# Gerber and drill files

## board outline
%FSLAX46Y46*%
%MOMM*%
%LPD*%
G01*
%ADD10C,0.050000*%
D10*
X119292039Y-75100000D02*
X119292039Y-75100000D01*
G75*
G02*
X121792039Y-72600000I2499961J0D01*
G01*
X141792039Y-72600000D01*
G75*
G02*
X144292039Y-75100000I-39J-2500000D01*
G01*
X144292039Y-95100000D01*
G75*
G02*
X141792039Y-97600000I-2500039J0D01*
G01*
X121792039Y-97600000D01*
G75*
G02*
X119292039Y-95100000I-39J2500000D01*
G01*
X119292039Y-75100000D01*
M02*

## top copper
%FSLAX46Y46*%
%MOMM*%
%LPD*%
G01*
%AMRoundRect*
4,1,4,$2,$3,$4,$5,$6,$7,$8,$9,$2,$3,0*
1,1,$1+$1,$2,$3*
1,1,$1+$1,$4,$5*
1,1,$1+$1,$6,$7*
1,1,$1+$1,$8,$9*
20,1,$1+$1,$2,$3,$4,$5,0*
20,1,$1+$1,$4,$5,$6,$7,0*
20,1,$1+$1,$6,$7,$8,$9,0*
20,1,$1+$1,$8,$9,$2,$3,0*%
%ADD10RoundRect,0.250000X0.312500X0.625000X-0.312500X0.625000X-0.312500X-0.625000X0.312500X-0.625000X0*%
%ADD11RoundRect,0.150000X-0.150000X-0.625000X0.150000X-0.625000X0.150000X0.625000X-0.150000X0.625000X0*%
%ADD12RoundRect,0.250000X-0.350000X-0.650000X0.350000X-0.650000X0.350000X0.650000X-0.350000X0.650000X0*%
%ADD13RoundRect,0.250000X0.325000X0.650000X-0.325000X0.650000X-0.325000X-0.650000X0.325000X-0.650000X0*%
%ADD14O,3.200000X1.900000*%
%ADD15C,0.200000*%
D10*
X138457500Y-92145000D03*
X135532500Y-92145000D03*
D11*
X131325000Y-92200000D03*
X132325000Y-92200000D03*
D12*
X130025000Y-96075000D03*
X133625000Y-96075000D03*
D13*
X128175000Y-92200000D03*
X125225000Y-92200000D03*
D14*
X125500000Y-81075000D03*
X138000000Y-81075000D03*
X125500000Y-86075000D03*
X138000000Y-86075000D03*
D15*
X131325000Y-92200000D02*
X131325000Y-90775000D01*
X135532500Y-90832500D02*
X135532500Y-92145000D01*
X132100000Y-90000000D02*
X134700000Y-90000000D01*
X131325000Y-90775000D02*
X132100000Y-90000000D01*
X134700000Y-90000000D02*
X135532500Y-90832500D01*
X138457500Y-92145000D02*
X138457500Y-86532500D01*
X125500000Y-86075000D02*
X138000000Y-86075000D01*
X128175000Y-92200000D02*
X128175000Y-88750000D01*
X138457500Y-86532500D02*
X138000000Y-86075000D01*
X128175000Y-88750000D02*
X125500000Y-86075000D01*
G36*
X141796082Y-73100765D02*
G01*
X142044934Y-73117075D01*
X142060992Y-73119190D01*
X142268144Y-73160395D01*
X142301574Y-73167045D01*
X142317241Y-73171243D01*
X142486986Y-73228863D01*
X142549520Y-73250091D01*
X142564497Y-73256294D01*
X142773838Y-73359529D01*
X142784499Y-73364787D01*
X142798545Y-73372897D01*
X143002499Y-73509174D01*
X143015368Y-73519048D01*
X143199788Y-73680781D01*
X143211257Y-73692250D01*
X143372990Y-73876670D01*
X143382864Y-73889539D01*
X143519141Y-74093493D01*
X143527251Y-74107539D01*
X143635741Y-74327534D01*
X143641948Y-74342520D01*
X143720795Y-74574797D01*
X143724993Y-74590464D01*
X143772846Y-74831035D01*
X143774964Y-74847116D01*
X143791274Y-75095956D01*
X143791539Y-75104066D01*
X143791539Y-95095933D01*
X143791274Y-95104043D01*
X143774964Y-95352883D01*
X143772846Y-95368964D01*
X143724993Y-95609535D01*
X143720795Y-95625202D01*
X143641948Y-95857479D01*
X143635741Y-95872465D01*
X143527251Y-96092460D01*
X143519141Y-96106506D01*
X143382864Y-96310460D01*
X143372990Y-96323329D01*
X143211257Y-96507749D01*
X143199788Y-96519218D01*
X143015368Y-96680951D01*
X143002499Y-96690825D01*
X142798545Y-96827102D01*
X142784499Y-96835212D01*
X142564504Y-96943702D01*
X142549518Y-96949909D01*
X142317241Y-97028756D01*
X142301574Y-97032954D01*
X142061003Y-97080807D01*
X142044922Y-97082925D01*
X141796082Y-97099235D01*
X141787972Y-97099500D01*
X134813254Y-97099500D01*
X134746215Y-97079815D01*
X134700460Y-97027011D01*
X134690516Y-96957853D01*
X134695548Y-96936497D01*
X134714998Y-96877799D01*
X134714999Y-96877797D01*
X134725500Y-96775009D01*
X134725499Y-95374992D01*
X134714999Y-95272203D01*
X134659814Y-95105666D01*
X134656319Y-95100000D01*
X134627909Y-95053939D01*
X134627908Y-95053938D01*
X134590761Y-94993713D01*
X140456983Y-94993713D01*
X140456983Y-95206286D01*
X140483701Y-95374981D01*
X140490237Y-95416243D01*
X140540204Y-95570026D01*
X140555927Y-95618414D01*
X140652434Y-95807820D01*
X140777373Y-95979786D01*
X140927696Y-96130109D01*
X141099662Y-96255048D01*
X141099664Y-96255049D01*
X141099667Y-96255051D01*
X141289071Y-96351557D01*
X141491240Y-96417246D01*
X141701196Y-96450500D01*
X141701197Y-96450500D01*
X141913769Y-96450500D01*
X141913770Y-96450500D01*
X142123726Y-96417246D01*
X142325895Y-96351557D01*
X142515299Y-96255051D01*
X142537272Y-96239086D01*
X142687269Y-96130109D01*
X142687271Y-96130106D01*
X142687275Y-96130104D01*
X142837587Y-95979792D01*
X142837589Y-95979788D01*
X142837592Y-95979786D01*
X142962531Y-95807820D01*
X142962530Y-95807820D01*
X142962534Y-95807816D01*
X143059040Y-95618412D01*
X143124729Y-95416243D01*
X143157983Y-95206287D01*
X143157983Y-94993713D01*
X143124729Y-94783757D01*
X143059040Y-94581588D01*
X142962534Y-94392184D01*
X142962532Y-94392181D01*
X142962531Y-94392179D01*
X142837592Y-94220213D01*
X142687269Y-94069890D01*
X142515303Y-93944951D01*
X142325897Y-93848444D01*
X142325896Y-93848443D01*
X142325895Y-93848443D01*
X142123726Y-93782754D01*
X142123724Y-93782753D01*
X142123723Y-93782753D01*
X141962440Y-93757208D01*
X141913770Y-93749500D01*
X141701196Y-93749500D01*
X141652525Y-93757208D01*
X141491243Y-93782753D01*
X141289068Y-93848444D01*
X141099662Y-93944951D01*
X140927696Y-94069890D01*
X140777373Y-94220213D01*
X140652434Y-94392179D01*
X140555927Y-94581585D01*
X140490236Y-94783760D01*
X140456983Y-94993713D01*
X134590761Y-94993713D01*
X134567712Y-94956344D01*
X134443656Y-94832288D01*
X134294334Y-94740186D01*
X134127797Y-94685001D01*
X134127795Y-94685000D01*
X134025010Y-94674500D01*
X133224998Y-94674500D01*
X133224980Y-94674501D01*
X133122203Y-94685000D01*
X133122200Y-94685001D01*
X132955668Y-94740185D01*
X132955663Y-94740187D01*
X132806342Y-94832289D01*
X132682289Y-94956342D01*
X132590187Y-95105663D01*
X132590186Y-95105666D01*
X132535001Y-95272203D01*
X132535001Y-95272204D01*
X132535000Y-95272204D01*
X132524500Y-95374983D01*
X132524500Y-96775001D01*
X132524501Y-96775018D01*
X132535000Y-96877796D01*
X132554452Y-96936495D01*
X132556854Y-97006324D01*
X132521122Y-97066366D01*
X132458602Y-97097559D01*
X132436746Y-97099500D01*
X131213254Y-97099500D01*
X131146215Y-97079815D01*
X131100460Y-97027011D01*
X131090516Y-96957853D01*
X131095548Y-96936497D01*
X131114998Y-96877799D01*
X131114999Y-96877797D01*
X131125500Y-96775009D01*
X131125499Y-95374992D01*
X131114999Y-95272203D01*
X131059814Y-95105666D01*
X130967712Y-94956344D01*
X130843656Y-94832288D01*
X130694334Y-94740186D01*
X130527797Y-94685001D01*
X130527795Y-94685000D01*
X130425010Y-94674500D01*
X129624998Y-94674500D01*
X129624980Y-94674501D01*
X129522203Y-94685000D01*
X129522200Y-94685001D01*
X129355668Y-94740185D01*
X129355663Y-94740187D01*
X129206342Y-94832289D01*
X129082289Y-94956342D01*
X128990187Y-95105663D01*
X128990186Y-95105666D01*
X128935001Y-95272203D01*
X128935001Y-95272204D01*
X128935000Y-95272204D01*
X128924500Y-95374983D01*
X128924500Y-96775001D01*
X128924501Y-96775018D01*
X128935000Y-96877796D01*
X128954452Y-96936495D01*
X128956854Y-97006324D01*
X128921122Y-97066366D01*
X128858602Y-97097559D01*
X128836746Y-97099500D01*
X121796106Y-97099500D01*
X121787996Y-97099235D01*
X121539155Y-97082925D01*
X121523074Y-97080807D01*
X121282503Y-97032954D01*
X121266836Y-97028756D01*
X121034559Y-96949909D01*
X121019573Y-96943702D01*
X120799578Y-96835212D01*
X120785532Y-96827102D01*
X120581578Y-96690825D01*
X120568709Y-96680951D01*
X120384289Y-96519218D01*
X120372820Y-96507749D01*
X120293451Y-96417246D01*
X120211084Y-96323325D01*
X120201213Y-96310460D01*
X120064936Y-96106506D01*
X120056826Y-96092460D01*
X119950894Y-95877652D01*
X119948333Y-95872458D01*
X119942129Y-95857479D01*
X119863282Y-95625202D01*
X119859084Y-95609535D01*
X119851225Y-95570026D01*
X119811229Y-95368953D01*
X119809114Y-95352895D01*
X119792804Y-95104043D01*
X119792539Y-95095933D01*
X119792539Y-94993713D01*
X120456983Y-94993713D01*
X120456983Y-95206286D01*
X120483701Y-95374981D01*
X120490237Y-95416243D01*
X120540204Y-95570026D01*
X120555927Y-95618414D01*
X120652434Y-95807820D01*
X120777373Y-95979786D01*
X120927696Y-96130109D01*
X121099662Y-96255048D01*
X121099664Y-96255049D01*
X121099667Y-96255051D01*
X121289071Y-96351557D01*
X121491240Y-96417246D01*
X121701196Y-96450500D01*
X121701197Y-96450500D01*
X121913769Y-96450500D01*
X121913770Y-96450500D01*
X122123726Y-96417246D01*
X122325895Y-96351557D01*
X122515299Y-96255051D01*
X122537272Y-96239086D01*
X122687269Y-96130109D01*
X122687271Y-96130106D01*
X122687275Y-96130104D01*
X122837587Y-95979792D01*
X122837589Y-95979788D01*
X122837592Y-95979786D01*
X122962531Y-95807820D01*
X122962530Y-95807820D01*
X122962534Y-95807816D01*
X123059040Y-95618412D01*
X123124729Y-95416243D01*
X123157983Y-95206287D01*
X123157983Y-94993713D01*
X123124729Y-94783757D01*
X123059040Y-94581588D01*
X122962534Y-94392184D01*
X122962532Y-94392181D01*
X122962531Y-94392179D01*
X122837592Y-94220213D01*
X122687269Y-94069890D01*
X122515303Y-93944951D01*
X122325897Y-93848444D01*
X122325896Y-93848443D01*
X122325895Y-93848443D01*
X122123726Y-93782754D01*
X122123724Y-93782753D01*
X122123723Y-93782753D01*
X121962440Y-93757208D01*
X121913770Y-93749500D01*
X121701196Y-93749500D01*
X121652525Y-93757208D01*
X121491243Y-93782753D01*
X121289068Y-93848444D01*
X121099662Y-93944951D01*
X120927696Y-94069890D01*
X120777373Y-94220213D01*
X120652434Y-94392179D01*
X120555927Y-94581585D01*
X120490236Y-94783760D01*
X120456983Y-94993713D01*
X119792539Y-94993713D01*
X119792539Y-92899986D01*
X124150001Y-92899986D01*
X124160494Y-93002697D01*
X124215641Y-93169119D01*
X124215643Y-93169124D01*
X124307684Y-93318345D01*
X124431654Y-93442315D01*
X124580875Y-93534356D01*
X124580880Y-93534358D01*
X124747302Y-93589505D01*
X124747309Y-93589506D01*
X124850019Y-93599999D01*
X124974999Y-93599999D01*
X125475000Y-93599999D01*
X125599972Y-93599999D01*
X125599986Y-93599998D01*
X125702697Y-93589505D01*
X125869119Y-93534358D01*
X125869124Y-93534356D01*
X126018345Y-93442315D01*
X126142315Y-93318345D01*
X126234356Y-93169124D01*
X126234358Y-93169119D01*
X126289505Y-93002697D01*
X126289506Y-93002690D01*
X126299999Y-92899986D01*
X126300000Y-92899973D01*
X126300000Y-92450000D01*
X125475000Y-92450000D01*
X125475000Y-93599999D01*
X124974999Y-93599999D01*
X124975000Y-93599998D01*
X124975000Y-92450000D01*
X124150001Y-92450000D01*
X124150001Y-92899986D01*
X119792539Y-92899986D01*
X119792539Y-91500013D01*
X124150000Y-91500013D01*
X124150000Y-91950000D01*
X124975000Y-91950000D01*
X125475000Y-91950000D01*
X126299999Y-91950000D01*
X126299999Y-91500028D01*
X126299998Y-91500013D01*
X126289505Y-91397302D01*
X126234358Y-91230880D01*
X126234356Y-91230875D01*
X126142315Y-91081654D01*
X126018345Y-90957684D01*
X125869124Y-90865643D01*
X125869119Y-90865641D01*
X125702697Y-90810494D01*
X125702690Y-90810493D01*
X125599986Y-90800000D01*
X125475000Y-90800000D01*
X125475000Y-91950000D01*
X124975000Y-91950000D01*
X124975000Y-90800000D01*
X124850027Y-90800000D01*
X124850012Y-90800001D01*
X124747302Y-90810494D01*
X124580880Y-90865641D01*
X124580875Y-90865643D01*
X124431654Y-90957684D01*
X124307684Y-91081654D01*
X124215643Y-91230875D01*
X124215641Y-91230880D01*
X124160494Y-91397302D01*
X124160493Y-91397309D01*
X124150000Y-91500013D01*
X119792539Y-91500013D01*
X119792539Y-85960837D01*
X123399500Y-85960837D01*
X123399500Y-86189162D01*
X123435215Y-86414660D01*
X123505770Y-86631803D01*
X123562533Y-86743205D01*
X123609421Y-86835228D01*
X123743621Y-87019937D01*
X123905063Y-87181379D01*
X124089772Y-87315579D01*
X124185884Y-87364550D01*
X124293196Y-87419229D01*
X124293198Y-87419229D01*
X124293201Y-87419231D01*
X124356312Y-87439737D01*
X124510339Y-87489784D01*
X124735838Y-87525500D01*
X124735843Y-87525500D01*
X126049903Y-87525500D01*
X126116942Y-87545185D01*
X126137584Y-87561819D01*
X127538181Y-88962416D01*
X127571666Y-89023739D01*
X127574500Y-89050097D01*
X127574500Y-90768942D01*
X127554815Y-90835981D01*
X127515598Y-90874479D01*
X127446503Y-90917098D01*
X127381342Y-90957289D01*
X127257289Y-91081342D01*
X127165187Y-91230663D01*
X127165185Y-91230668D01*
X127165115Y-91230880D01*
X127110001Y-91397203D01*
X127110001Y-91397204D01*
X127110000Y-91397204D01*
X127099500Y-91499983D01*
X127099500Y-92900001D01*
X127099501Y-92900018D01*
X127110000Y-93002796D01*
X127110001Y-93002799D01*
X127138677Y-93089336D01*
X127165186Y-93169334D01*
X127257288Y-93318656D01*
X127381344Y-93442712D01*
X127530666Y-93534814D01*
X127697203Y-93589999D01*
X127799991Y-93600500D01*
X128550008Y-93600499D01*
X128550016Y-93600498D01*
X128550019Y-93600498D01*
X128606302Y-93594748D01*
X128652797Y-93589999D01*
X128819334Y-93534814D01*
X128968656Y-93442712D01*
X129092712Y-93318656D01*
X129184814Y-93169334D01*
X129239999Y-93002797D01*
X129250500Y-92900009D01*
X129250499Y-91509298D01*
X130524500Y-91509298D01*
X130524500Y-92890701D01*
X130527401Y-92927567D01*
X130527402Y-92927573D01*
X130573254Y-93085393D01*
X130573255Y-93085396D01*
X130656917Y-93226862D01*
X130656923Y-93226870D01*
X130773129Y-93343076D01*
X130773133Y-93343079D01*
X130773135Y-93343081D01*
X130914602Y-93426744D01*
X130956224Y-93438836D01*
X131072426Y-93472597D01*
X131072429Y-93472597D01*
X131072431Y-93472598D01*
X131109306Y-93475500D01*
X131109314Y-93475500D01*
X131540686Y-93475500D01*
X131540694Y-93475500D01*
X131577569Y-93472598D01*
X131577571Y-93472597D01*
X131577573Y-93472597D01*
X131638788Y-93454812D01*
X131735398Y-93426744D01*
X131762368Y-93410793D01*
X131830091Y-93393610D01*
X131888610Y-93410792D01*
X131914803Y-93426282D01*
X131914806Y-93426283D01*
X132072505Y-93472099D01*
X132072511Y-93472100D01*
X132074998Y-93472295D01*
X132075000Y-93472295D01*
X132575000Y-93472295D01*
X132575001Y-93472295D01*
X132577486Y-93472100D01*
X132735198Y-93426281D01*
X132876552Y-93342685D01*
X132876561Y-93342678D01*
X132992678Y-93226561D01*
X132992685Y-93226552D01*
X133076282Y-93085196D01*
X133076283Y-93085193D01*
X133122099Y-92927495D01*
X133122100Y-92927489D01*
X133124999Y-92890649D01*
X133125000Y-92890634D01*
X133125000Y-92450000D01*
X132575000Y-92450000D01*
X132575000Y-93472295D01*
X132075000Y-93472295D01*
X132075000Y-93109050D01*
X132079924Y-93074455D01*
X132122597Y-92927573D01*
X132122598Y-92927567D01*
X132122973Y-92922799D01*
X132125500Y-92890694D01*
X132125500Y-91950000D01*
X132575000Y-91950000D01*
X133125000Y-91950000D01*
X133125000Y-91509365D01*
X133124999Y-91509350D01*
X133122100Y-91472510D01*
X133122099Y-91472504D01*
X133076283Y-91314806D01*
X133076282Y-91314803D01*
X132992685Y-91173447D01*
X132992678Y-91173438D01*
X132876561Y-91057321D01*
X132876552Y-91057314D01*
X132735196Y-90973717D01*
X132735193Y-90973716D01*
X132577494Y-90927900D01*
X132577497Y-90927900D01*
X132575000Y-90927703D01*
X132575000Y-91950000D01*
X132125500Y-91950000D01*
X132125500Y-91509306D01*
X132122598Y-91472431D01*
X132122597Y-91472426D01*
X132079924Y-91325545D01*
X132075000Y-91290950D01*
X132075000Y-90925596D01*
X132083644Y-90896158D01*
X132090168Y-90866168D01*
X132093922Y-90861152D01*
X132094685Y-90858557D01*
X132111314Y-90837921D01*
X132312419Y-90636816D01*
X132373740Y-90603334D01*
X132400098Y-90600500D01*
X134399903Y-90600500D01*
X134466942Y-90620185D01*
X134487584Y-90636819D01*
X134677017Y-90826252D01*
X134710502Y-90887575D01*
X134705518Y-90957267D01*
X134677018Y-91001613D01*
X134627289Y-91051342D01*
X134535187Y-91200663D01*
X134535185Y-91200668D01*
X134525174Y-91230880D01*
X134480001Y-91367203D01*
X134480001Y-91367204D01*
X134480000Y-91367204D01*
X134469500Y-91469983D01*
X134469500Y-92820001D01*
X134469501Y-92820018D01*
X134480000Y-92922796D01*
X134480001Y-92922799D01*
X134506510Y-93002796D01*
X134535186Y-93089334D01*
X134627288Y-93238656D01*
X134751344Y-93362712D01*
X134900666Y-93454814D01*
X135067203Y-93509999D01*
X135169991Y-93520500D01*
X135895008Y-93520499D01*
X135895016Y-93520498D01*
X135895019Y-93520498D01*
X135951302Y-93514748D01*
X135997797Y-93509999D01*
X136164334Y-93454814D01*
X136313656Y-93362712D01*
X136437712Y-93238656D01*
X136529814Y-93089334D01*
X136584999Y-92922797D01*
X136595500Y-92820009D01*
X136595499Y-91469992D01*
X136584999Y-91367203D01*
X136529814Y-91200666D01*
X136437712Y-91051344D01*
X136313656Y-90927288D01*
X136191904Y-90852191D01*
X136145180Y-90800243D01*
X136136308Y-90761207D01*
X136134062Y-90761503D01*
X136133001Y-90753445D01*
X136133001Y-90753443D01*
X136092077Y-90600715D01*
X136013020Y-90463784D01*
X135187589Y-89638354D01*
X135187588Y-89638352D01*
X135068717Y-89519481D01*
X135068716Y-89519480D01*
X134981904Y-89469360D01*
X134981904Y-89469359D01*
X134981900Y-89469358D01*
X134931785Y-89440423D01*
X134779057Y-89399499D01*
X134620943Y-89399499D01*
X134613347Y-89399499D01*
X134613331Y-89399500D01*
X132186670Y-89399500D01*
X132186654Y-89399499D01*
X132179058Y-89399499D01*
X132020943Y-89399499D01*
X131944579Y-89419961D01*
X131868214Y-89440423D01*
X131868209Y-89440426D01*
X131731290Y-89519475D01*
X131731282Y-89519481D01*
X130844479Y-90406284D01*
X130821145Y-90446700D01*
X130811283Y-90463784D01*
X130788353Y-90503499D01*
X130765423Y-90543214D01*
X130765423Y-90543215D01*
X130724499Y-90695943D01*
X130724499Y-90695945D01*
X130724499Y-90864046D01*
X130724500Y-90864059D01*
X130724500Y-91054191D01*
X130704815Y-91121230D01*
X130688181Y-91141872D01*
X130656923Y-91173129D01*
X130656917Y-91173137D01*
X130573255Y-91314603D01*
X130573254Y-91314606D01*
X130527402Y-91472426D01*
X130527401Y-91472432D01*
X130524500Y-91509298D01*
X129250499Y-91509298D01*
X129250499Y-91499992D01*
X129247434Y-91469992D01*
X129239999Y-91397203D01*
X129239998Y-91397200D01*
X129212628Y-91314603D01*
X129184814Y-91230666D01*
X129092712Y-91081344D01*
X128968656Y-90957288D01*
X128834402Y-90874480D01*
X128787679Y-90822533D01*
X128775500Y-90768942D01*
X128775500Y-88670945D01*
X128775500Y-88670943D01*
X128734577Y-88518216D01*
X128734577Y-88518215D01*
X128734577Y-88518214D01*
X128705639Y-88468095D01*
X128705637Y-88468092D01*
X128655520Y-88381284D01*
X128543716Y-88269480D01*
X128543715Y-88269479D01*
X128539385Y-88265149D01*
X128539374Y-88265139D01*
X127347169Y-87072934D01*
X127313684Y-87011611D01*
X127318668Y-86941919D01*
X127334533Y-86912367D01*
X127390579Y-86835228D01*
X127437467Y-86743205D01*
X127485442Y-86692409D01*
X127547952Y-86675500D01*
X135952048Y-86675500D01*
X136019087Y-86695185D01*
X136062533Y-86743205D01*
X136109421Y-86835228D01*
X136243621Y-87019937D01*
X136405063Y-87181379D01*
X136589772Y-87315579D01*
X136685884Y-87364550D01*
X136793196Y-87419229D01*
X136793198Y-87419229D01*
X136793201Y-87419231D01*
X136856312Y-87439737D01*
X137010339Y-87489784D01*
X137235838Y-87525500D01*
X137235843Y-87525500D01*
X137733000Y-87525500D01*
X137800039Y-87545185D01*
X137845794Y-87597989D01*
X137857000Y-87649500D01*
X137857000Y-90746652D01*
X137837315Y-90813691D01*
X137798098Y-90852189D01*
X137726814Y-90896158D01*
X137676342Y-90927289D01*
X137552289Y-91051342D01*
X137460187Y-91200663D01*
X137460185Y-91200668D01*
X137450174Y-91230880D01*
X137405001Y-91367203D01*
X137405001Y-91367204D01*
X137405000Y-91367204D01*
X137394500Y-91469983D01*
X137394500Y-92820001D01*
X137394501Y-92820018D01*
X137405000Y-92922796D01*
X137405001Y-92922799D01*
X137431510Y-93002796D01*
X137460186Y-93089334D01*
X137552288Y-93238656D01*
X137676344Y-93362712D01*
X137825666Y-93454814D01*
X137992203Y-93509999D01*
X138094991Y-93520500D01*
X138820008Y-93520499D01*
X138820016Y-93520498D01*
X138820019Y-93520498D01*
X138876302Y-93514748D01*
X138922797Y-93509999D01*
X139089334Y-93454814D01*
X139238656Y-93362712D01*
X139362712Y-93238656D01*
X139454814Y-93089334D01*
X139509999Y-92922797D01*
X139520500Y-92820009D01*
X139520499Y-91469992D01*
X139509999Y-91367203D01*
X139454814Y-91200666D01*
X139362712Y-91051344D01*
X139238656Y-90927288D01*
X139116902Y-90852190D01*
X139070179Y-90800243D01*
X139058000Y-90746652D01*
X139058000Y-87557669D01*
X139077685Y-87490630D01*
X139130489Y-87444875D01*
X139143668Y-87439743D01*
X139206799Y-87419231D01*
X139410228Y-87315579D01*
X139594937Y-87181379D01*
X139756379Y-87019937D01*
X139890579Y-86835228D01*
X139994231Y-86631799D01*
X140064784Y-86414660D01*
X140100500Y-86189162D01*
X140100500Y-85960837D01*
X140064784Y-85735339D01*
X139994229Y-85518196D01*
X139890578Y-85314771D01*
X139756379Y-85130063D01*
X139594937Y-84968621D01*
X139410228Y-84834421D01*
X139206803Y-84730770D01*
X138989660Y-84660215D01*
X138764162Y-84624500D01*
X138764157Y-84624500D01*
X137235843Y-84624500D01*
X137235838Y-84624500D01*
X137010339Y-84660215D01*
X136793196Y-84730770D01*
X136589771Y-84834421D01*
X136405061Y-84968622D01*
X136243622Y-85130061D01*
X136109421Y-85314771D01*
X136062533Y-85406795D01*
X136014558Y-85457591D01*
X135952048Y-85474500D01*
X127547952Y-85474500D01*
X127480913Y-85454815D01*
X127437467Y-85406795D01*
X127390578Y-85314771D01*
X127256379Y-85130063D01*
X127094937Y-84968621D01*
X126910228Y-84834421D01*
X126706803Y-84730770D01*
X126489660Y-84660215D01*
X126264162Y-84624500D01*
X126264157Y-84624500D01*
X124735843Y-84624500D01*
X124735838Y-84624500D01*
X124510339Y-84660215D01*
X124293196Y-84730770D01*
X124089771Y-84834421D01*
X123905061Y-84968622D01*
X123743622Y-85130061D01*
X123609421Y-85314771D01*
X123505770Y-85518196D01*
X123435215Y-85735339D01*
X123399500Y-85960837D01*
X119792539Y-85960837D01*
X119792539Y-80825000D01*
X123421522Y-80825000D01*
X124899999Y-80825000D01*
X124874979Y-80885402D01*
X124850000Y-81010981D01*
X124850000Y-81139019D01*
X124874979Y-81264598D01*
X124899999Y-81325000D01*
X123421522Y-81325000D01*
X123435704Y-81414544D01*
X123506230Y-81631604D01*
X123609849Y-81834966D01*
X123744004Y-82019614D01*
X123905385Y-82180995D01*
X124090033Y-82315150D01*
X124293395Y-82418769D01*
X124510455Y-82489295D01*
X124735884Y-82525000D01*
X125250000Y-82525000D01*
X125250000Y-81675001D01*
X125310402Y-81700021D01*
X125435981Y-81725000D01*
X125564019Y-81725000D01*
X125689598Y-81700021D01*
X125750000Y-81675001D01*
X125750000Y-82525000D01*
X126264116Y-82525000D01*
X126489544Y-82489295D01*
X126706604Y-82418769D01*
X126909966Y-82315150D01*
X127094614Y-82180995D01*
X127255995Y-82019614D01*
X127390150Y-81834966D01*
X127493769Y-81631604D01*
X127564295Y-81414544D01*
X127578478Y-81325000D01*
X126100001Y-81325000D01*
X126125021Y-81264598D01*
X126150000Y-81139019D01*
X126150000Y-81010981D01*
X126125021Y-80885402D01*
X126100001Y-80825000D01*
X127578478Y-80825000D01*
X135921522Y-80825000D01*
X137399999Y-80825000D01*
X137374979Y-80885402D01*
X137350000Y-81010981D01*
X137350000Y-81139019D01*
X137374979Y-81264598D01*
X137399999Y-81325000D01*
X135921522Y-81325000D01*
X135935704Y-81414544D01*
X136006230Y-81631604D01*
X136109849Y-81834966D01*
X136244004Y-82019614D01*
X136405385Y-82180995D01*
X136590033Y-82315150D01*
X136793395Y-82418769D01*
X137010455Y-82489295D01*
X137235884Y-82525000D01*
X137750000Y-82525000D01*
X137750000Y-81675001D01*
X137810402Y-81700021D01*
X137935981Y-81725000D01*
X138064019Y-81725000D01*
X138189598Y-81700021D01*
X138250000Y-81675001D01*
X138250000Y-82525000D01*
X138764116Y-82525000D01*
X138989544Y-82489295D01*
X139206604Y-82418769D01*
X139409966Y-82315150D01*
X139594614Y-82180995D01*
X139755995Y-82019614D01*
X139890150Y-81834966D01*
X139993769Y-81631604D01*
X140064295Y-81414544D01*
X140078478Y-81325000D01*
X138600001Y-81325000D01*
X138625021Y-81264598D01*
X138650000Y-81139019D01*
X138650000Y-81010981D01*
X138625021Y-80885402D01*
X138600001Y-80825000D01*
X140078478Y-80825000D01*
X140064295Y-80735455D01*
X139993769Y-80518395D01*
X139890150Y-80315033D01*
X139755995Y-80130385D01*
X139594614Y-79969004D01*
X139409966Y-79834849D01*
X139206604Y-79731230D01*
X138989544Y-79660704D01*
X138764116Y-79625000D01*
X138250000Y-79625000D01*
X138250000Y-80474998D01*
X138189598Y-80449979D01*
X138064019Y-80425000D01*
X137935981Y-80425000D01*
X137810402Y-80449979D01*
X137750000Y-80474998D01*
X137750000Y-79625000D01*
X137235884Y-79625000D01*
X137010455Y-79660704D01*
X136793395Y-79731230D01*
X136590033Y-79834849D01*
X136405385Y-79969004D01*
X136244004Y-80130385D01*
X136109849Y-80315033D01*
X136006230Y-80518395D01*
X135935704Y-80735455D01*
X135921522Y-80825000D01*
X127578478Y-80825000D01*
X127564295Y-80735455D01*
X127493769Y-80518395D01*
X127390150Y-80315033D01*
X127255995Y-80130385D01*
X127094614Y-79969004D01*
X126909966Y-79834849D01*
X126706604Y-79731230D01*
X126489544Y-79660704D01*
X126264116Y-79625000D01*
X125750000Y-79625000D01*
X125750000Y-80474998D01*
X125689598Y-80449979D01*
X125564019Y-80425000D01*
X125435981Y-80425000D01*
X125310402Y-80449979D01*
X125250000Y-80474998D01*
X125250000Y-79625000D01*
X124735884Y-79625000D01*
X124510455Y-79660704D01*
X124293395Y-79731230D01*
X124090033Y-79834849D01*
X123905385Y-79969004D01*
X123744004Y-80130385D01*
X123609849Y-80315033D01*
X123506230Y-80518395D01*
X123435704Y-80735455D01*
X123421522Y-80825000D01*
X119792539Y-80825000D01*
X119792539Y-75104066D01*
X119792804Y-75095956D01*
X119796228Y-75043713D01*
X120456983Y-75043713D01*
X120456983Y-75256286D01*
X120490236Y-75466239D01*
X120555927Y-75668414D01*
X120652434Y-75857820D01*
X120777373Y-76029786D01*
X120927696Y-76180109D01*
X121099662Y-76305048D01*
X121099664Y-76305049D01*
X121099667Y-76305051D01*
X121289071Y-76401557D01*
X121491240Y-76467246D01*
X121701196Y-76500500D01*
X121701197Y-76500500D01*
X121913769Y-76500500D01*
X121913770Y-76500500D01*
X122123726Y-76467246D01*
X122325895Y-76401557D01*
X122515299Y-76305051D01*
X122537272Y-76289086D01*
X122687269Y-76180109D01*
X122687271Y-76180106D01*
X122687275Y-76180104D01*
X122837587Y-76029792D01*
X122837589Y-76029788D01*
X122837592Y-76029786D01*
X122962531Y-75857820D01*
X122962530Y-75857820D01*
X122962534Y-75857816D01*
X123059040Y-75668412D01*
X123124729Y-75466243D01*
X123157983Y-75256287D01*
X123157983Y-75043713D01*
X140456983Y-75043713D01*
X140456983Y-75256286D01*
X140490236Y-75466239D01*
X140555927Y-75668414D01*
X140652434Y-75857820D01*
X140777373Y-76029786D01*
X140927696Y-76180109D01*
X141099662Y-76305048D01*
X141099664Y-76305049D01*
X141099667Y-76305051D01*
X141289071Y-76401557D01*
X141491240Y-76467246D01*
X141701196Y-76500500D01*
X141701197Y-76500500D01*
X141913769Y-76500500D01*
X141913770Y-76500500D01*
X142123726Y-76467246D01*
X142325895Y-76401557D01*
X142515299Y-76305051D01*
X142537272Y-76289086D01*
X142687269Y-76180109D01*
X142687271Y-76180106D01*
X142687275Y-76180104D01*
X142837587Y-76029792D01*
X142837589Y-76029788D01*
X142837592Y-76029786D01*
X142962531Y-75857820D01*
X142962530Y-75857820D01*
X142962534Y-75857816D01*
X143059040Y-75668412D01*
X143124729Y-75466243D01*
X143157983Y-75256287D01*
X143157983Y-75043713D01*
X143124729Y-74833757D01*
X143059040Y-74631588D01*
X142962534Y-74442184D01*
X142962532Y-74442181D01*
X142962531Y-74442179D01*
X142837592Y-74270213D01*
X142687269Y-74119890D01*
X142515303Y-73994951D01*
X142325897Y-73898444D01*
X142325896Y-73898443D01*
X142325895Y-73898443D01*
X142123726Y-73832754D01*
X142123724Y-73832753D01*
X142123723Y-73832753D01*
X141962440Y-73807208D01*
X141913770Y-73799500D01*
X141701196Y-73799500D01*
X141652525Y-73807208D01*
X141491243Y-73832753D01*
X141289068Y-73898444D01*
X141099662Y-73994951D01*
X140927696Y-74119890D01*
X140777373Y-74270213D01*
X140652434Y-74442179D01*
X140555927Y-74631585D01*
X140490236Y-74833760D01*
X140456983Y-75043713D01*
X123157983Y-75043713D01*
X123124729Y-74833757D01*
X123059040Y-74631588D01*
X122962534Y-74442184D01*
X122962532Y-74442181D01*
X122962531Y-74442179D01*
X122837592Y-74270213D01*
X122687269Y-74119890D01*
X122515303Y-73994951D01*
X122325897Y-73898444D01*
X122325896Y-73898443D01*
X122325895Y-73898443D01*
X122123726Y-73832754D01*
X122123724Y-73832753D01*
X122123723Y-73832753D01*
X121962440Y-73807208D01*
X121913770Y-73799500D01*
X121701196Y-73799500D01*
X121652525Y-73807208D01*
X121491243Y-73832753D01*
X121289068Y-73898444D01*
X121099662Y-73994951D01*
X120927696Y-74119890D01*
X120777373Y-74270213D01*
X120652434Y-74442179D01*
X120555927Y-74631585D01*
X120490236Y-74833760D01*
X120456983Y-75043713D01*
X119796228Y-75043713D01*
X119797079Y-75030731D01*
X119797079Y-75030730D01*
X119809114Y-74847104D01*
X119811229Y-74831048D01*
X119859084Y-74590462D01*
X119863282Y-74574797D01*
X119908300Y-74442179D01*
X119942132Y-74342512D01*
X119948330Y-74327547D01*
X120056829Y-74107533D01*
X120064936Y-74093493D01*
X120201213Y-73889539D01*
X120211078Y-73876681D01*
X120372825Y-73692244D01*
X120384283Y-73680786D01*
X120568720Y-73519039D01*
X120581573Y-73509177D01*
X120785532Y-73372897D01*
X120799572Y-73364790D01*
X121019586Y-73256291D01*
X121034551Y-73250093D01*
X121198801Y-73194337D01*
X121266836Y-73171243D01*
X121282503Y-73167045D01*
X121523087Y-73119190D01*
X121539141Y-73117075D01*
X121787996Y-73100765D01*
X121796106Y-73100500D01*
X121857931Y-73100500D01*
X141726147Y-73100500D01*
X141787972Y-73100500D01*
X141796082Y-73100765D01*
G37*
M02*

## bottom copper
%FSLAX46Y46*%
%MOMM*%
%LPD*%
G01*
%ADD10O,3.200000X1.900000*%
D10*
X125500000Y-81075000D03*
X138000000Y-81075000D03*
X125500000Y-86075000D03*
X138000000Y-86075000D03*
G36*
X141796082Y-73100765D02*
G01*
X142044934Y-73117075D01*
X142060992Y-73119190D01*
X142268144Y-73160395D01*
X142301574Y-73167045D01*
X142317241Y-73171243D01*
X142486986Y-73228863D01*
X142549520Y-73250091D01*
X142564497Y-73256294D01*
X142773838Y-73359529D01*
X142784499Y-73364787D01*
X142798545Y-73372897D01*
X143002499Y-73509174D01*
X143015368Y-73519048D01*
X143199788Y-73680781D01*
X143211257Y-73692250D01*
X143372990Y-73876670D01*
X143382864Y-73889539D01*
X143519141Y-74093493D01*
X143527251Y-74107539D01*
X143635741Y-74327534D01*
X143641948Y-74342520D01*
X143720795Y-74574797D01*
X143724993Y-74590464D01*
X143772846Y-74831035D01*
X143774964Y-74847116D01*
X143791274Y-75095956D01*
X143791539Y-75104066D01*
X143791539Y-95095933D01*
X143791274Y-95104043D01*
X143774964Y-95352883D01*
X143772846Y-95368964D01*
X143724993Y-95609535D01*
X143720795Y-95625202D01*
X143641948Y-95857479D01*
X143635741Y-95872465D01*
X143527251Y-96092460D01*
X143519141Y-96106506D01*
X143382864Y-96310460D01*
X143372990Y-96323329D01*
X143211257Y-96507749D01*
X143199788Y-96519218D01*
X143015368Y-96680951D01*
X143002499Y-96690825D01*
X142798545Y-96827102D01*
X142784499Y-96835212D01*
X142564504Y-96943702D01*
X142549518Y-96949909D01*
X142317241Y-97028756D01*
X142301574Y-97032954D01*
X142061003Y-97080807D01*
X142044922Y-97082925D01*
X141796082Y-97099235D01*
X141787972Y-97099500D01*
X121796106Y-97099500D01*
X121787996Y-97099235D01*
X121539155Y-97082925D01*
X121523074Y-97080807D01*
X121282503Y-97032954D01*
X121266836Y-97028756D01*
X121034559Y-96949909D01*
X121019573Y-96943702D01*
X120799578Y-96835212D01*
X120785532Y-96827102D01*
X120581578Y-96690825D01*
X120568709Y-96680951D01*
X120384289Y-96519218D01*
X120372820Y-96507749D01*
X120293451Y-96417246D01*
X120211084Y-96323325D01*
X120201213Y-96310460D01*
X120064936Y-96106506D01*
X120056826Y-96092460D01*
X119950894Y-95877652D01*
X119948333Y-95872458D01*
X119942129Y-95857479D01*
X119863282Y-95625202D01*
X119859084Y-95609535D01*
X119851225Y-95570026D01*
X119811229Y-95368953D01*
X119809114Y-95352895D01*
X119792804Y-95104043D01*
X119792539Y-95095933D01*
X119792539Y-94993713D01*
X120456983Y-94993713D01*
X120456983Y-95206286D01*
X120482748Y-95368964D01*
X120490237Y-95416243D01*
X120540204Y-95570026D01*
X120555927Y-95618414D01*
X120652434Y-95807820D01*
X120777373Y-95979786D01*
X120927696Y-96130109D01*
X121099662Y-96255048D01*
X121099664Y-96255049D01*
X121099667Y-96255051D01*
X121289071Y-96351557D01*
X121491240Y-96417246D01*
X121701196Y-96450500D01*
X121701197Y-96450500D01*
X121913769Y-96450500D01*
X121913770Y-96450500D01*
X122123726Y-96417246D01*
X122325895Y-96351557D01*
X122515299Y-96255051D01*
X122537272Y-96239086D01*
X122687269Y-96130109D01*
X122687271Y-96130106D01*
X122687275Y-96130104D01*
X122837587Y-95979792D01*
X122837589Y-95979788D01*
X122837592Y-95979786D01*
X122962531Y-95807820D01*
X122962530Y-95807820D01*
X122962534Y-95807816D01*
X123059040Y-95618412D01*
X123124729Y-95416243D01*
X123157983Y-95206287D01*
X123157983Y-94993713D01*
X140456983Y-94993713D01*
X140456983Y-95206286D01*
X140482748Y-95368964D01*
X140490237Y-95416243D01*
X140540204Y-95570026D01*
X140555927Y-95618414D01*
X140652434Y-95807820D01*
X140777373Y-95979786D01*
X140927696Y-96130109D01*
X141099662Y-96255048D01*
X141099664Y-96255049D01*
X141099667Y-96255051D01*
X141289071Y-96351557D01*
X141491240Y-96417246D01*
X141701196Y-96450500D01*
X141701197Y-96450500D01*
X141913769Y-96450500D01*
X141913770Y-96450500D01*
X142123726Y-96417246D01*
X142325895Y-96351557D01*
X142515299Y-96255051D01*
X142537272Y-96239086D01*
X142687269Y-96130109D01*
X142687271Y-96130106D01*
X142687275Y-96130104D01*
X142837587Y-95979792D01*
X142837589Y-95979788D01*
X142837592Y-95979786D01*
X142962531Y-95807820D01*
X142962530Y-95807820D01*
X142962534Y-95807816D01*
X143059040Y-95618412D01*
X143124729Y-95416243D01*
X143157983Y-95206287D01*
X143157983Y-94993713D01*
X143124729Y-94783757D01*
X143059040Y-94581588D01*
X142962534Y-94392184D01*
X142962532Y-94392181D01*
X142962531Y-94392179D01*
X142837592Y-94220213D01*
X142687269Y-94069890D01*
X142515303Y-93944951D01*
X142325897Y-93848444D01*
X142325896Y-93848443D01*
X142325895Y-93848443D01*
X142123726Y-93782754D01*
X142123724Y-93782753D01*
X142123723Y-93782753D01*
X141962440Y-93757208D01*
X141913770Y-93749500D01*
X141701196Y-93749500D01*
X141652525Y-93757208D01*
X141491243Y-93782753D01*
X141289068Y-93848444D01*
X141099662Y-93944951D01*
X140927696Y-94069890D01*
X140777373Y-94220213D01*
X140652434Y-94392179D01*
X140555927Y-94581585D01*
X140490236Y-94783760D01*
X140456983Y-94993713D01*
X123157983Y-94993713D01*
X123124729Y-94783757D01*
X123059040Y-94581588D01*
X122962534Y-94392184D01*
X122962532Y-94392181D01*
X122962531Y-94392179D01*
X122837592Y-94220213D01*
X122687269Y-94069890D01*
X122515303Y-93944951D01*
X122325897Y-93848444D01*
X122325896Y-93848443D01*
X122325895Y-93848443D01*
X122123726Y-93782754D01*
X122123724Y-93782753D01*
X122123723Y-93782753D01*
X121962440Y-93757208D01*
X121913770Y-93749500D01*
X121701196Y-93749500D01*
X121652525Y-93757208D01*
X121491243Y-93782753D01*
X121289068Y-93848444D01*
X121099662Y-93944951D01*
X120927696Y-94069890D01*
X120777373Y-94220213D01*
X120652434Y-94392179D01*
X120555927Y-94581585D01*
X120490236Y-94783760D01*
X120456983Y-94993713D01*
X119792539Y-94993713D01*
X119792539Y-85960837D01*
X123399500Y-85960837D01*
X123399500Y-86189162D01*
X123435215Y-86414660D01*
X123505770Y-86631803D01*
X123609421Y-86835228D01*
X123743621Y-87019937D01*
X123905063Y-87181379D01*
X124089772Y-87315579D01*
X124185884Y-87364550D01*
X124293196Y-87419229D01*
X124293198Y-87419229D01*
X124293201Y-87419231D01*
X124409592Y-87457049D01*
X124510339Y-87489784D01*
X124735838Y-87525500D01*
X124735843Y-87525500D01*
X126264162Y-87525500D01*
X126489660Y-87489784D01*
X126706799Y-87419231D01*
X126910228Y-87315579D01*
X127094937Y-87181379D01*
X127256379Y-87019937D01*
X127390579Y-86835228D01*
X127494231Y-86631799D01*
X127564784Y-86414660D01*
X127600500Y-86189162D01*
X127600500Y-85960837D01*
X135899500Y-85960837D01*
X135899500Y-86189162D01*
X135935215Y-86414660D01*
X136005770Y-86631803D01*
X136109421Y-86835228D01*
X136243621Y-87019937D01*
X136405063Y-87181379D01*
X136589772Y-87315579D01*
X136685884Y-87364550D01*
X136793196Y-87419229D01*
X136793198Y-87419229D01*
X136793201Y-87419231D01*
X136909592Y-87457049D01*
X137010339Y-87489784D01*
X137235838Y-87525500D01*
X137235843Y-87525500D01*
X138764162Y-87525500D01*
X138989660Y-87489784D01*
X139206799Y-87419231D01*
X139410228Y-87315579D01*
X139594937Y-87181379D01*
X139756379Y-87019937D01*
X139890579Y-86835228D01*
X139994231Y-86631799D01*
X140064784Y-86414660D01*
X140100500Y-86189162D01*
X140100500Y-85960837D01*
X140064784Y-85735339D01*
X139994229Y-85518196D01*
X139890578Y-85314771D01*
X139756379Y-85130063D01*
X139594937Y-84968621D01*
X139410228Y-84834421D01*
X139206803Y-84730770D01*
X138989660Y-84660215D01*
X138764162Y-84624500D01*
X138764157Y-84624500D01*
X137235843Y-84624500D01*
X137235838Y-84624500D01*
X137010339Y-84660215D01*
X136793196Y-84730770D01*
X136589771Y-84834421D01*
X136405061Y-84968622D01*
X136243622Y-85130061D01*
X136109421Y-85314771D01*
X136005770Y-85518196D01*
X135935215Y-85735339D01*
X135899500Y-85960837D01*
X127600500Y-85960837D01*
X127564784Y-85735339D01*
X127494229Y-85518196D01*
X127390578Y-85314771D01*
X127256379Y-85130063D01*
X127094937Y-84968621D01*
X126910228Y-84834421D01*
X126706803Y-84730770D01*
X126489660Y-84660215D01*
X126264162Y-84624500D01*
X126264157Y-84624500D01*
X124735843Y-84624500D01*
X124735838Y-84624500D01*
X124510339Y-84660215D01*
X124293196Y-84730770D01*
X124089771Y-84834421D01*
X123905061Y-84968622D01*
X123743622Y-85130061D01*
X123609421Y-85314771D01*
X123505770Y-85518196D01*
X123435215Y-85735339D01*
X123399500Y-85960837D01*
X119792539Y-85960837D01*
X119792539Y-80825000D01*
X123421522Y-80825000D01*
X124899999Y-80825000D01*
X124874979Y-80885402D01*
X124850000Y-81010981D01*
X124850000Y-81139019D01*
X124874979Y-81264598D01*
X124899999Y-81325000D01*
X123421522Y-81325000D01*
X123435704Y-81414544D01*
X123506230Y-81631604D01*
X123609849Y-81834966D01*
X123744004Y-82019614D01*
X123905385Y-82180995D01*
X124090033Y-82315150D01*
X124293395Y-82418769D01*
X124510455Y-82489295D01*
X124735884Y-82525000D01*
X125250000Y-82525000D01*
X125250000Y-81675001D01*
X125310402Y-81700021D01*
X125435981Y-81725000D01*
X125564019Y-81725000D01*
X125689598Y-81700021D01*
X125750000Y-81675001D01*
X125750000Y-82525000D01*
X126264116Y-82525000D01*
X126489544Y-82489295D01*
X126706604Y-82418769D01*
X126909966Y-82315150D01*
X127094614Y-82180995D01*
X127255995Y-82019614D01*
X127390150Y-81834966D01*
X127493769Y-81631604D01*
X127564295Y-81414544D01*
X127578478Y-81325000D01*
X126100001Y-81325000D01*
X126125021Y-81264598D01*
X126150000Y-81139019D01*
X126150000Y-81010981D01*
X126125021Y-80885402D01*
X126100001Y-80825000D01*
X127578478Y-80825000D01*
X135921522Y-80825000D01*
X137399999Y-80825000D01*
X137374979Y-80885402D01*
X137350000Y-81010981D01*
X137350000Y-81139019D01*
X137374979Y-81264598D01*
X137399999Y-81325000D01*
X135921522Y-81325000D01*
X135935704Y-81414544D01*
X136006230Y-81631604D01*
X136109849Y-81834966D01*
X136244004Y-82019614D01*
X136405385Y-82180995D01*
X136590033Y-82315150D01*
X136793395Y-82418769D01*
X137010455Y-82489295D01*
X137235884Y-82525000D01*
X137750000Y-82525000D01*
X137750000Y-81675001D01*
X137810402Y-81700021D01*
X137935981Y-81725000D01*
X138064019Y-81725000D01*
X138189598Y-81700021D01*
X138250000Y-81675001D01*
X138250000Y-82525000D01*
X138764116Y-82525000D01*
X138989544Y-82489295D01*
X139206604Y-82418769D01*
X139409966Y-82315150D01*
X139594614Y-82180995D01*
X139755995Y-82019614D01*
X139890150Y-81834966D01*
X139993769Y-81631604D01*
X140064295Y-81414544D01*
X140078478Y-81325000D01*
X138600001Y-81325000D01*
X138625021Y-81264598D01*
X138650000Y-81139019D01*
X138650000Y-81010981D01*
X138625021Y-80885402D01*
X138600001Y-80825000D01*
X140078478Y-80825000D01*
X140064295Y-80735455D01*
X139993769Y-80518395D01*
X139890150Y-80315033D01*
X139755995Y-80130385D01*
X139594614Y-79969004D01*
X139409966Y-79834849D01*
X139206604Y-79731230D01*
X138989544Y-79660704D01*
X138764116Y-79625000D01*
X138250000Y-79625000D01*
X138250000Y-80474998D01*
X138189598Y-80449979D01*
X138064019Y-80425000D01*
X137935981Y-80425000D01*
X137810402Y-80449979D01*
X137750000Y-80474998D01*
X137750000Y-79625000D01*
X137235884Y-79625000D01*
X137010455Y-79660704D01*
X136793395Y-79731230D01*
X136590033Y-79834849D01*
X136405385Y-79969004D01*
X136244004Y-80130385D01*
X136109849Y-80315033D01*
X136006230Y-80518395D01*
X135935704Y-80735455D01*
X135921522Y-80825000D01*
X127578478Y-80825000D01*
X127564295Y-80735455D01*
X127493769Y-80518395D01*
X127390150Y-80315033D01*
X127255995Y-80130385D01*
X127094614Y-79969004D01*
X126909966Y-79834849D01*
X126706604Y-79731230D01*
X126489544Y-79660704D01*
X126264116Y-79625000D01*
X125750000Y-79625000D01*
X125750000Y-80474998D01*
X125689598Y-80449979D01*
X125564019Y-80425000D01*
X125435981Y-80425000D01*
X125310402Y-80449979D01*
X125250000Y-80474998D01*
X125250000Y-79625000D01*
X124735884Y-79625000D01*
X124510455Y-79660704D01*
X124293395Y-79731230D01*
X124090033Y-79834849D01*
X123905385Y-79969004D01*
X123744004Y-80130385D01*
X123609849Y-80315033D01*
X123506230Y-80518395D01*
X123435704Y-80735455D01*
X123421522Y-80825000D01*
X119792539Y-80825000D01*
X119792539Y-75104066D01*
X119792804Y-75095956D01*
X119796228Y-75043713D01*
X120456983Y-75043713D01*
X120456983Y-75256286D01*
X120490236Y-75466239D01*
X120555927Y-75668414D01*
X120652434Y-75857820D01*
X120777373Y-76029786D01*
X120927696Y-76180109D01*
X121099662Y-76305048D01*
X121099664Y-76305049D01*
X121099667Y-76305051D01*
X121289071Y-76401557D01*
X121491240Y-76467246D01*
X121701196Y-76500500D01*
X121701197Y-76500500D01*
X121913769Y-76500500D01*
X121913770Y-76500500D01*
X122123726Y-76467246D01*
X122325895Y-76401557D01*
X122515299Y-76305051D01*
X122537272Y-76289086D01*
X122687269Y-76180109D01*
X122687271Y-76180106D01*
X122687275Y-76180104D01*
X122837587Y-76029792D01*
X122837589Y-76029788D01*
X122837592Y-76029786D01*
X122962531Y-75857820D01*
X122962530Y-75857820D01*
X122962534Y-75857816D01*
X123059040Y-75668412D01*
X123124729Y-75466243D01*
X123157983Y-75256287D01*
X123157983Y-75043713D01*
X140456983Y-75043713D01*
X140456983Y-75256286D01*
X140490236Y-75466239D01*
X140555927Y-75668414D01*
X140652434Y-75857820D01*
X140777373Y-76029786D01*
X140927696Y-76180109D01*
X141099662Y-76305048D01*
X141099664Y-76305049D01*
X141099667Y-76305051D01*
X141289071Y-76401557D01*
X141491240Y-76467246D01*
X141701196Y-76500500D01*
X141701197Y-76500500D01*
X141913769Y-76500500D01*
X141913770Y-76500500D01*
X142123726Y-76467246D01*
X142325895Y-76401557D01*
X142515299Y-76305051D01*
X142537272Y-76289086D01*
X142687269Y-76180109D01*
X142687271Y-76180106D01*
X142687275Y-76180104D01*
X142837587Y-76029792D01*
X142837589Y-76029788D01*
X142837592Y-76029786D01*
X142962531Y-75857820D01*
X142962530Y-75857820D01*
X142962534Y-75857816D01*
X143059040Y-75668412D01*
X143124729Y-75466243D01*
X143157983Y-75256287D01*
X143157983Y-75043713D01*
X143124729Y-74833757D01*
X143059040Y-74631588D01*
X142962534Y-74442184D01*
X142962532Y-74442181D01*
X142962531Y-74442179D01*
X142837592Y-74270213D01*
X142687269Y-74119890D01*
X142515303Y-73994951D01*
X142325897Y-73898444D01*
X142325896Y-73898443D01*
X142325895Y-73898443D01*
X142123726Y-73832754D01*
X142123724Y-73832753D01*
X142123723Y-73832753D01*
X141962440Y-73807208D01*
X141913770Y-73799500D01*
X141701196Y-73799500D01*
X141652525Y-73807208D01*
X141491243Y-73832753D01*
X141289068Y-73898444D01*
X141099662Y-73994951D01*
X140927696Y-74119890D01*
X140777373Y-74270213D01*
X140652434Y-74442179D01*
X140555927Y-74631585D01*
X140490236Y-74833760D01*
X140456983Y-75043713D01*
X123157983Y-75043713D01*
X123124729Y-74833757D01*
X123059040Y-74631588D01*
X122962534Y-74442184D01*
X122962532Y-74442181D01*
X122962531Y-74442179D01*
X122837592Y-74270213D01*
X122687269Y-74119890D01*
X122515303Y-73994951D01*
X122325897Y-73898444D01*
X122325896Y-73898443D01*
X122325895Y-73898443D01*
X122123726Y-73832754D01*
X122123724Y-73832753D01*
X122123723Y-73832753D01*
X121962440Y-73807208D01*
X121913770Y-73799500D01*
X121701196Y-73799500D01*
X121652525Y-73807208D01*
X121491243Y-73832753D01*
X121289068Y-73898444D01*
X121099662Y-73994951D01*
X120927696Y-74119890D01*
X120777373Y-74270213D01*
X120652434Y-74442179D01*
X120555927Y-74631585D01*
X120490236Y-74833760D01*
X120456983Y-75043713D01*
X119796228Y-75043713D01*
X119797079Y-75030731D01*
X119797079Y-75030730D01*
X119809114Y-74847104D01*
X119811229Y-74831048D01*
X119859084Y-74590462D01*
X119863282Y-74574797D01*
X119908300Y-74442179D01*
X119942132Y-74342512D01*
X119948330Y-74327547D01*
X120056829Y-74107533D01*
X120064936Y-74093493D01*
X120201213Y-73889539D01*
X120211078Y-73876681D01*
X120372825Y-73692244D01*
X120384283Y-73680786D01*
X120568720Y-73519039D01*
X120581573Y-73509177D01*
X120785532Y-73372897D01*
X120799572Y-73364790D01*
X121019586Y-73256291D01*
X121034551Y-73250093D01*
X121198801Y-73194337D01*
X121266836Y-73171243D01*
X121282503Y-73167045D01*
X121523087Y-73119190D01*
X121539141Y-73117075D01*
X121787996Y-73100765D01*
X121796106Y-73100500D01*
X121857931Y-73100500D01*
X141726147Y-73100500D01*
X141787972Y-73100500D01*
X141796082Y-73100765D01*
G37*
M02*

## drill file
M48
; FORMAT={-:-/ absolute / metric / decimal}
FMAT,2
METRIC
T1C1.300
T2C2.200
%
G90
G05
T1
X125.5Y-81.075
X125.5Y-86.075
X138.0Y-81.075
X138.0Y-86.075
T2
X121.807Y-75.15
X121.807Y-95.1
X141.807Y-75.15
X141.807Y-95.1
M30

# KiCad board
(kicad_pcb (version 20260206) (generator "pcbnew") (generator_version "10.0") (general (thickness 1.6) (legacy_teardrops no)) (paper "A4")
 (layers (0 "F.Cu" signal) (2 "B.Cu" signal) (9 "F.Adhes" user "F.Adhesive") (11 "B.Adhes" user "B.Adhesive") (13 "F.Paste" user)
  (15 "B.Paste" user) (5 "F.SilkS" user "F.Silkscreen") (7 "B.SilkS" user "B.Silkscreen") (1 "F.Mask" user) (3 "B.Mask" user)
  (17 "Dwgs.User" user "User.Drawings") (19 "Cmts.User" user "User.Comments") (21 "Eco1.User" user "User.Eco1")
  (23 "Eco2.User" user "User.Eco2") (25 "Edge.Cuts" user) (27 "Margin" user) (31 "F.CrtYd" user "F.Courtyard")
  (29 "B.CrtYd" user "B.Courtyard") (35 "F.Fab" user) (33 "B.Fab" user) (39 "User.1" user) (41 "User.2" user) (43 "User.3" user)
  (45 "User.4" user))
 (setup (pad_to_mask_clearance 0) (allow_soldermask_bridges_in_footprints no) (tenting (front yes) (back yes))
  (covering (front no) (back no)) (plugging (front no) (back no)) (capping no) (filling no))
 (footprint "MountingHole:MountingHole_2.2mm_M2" (layer "F.Cu") (at 141.807483 95.1)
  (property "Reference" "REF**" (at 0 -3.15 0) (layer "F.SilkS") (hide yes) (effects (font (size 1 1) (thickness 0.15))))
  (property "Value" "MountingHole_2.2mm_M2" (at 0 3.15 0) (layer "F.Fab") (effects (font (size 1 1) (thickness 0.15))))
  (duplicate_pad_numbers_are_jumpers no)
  (pad "" np_thru_hole circle (at 0 0) (size 2.2 2.2) (drill 2.2) (layers "*.Cu" "*.Mask")))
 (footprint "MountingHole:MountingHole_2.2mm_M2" (layer "F.Cu") (at 121.807483 95.1)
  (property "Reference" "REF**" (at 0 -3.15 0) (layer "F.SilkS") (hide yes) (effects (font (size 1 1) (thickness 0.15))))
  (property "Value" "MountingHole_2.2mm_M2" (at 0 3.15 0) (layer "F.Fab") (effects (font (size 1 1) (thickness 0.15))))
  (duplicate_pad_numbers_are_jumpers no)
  (pad "" np_thru_hole circle (at 0 0) (size 2.2 2.2) (drill 2.2) (layers "*.Cu" "*.Mask")))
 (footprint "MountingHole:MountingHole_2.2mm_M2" (layer "F.Cu") (at 141.807483 75.15)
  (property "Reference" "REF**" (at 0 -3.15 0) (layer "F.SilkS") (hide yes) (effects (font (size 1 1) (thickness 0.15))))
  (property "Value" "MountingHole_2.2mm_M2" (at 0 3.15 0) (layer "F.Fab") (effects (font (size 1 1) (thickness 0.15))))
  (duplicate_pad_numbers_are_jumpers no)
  (pad "" np_thru_hole circle (at 0 0) (size 2.2 2.2) (drill 2.2) (layers "*.Cu" "*.Mask")))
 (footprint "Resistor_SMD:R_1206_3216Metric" (layer "F.Cu") (at 136.995 92.145 180)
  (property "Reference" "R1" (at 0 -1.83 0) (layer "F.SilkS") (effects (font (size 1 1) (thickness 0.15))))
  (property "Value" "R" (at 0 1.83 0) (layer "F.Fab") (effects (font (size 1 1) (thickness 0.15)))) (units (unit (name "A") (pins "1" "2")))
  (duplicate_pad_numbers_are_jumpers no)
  (pad "1" smd roundrect (at -1.4625 0 180) (size 1.125 1.75) (layers "F.Cu" "F.Mask" "F.Paste") (roundrect_rratio 0.222222) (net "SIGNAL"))
  (pad "2" smd roundrect (at 1.4625 0 180) (size 1.125 1.75) (layers "F.Cu" "F.Mask" "F.Paste") (roundrect_rratio 0.222222)
   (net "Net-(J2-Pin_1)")))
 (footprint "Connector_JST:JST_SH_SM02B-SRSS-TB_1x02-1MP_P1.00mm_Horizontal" (layer "F.Cu") (at 131.825 94.2)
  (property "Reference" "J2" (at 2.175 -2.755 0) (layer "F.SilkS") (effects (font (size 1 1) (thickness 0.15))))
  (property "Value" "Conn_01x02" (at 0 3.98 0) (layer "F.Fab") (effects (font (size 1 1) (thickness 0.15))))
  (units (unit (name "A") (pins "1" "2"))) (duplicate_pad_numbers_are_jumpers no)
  (pad "1" smd roundrect (at -0.5 -2) (size 0.6 1.55) (layers "F.Cu" "F.Mask" "F.Paste") (roundrect_rratio 0.25) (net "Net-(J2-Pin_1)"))
  (pad "2" smd roundrect (at 0.5 -2) (size 0.6 1.55) (layers "F.Cu" "F.Mask" "F.Paste") (roundrect_rratio 0.25) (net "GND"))
  (pad "MP" smd roundrect (at -1.8 1.875) (size 1.2 1.8) (layers "F.Cu" "F.Mask" "F.Paste") (roundrect_rratio 0.208333))
  (pad "MP" smd roundrect (at 1.8 1.875) (size 1.2 1.8) (layers "F.Cu" "F.Mask" "F.Paste") (roundrect_rratio 0.208333)))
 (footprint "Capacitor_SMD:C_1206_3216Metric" (layer "F.Cu") (at 126.7 92.2 180)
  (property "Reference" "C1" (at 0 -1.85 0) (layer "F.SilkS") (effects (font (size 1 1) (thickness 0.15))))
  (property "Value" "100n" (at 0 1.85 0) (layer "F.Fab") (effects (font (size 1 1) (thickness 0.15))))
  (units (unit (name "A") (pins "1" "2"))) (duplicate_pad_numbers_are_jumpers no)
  (pad "1" smd roundrect (at -1.475 0 180) (size 1.15 1.8) (layers "F.Cu" "F.Mask" "F.Paste") (roundrect_rratio 0.217391) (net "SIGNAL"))
  (pad "2" smd roundrect (at 1.475 0 180) (size 1.15 1.8) (layers "F.Cu" "F.Mask" "F.Paste") (roundrect_rratio 0.217391) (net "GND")))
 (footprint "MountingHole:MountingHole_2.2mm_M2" (layer "F.Cu") (at 121.807483 75.15)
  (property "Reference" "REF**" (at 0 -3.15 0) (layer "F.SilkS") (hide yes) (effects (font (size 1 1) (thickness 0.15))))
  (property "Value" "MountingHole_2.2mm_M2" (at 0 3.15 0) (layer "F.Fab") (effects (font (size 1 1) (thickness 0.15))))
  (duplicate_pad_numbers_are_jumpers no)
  (pad "" np_thru_hole circle (at 0 0) (size 2.2 2.2) (drill 2.2) (layers "*.Cu" "*.Mask")))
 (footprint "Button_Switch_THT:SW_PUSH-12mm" (layer "F.Cu") (at 125.5 81.075)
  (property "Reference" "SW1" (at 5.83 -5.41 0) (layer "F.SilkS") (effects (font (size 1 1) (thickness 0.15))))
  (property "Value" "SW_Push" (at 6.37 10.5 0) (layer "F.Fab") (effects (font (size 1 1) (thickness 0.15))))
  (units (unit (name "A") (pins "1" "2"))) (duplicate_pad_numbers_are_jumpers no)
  (pad "1" thru_hole oval (at 0 0) (size 3.2 1.9) (drill 1.3) (layers "*.Cu" "*.Mask") (remove_unused_layers no) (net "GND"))
  (pad "1" thru_hole oval (at 12.5 0) (size 3.2 1.9) (drill 1.3) (layers "*.Cu" "*.Mask") (remove_unused_layers no) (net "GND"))
  (pad "2" thru_hole oval (at 0 5) (size 3.2 1.9) (drill 1.3) (layers "*.Cu" "*.Mask") (remove_unused_layers no) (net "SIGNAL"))
  (pad "2" thru_hole oval (at 12.5 5) (size 3.2 1.9) (drill 1.3) (layers "*.Cu" "*.Mask") (remove_unused_layers no) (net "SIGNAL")))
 (gr_rect (start 119.292039 72.6) (end 144.292039 97.6) (radius 2.5) (stroke (width 0.05) (type solid)) (fill no) (layer "Edge.Cuts"))
 (segment (start 131.325 92.2) (end 131.325 90.775) (width 0.2) (layer "F.Cu") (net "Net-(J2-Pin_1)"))
 (segment (start 135.5325 90.8325) (end 135.5325 92.145) (width 0.2) (layer "F.Cu") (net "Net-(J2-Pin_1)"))
 (segment (start 132.1 90) (end 134.7 90) (width 0.2) (layer "F.Cu") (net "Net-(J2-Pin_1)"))
 (segment (start 131.325 90.775) (end 132.1 90) (width 0.2) (layer "F.Cu") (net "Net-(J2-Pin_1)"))
 (segment (start 134.7 90) (end 135.5325 90.8325) (width 0.2) (layer "F.Cu") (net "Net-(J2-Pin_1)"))
 (segment (start 138.4575 92.145) (end 138.4575 86.5325) (width 0.2) (layer "F.Cu") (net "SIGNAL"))
 (segment (start 125.5 86.075) (end 138 86.075) (width 0.2) (layer "F.Cu") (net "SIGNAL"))
 (segment (start 128.175 92.2) (end 128.175 88.75) (width 0.2) (layer "F.Cu") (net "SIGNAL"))
 (segment (start 138.4575 86.5325) (end 138 86.075) (width 0.2) (layer "F.Cu") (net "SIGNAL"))
 (segment (start 128.175 88.75) (end 125.5 86.075) (width 0.2) (layer "F.Cu") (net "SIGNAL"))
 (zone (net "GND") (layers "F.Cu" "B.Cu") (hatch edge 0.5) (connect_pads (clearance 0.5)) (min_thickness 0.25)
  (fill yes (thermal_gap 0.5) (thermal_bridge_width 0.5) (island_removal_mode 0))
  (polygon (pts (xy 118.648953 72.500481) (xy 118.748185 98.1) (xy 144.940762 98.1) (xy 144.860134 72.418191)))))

